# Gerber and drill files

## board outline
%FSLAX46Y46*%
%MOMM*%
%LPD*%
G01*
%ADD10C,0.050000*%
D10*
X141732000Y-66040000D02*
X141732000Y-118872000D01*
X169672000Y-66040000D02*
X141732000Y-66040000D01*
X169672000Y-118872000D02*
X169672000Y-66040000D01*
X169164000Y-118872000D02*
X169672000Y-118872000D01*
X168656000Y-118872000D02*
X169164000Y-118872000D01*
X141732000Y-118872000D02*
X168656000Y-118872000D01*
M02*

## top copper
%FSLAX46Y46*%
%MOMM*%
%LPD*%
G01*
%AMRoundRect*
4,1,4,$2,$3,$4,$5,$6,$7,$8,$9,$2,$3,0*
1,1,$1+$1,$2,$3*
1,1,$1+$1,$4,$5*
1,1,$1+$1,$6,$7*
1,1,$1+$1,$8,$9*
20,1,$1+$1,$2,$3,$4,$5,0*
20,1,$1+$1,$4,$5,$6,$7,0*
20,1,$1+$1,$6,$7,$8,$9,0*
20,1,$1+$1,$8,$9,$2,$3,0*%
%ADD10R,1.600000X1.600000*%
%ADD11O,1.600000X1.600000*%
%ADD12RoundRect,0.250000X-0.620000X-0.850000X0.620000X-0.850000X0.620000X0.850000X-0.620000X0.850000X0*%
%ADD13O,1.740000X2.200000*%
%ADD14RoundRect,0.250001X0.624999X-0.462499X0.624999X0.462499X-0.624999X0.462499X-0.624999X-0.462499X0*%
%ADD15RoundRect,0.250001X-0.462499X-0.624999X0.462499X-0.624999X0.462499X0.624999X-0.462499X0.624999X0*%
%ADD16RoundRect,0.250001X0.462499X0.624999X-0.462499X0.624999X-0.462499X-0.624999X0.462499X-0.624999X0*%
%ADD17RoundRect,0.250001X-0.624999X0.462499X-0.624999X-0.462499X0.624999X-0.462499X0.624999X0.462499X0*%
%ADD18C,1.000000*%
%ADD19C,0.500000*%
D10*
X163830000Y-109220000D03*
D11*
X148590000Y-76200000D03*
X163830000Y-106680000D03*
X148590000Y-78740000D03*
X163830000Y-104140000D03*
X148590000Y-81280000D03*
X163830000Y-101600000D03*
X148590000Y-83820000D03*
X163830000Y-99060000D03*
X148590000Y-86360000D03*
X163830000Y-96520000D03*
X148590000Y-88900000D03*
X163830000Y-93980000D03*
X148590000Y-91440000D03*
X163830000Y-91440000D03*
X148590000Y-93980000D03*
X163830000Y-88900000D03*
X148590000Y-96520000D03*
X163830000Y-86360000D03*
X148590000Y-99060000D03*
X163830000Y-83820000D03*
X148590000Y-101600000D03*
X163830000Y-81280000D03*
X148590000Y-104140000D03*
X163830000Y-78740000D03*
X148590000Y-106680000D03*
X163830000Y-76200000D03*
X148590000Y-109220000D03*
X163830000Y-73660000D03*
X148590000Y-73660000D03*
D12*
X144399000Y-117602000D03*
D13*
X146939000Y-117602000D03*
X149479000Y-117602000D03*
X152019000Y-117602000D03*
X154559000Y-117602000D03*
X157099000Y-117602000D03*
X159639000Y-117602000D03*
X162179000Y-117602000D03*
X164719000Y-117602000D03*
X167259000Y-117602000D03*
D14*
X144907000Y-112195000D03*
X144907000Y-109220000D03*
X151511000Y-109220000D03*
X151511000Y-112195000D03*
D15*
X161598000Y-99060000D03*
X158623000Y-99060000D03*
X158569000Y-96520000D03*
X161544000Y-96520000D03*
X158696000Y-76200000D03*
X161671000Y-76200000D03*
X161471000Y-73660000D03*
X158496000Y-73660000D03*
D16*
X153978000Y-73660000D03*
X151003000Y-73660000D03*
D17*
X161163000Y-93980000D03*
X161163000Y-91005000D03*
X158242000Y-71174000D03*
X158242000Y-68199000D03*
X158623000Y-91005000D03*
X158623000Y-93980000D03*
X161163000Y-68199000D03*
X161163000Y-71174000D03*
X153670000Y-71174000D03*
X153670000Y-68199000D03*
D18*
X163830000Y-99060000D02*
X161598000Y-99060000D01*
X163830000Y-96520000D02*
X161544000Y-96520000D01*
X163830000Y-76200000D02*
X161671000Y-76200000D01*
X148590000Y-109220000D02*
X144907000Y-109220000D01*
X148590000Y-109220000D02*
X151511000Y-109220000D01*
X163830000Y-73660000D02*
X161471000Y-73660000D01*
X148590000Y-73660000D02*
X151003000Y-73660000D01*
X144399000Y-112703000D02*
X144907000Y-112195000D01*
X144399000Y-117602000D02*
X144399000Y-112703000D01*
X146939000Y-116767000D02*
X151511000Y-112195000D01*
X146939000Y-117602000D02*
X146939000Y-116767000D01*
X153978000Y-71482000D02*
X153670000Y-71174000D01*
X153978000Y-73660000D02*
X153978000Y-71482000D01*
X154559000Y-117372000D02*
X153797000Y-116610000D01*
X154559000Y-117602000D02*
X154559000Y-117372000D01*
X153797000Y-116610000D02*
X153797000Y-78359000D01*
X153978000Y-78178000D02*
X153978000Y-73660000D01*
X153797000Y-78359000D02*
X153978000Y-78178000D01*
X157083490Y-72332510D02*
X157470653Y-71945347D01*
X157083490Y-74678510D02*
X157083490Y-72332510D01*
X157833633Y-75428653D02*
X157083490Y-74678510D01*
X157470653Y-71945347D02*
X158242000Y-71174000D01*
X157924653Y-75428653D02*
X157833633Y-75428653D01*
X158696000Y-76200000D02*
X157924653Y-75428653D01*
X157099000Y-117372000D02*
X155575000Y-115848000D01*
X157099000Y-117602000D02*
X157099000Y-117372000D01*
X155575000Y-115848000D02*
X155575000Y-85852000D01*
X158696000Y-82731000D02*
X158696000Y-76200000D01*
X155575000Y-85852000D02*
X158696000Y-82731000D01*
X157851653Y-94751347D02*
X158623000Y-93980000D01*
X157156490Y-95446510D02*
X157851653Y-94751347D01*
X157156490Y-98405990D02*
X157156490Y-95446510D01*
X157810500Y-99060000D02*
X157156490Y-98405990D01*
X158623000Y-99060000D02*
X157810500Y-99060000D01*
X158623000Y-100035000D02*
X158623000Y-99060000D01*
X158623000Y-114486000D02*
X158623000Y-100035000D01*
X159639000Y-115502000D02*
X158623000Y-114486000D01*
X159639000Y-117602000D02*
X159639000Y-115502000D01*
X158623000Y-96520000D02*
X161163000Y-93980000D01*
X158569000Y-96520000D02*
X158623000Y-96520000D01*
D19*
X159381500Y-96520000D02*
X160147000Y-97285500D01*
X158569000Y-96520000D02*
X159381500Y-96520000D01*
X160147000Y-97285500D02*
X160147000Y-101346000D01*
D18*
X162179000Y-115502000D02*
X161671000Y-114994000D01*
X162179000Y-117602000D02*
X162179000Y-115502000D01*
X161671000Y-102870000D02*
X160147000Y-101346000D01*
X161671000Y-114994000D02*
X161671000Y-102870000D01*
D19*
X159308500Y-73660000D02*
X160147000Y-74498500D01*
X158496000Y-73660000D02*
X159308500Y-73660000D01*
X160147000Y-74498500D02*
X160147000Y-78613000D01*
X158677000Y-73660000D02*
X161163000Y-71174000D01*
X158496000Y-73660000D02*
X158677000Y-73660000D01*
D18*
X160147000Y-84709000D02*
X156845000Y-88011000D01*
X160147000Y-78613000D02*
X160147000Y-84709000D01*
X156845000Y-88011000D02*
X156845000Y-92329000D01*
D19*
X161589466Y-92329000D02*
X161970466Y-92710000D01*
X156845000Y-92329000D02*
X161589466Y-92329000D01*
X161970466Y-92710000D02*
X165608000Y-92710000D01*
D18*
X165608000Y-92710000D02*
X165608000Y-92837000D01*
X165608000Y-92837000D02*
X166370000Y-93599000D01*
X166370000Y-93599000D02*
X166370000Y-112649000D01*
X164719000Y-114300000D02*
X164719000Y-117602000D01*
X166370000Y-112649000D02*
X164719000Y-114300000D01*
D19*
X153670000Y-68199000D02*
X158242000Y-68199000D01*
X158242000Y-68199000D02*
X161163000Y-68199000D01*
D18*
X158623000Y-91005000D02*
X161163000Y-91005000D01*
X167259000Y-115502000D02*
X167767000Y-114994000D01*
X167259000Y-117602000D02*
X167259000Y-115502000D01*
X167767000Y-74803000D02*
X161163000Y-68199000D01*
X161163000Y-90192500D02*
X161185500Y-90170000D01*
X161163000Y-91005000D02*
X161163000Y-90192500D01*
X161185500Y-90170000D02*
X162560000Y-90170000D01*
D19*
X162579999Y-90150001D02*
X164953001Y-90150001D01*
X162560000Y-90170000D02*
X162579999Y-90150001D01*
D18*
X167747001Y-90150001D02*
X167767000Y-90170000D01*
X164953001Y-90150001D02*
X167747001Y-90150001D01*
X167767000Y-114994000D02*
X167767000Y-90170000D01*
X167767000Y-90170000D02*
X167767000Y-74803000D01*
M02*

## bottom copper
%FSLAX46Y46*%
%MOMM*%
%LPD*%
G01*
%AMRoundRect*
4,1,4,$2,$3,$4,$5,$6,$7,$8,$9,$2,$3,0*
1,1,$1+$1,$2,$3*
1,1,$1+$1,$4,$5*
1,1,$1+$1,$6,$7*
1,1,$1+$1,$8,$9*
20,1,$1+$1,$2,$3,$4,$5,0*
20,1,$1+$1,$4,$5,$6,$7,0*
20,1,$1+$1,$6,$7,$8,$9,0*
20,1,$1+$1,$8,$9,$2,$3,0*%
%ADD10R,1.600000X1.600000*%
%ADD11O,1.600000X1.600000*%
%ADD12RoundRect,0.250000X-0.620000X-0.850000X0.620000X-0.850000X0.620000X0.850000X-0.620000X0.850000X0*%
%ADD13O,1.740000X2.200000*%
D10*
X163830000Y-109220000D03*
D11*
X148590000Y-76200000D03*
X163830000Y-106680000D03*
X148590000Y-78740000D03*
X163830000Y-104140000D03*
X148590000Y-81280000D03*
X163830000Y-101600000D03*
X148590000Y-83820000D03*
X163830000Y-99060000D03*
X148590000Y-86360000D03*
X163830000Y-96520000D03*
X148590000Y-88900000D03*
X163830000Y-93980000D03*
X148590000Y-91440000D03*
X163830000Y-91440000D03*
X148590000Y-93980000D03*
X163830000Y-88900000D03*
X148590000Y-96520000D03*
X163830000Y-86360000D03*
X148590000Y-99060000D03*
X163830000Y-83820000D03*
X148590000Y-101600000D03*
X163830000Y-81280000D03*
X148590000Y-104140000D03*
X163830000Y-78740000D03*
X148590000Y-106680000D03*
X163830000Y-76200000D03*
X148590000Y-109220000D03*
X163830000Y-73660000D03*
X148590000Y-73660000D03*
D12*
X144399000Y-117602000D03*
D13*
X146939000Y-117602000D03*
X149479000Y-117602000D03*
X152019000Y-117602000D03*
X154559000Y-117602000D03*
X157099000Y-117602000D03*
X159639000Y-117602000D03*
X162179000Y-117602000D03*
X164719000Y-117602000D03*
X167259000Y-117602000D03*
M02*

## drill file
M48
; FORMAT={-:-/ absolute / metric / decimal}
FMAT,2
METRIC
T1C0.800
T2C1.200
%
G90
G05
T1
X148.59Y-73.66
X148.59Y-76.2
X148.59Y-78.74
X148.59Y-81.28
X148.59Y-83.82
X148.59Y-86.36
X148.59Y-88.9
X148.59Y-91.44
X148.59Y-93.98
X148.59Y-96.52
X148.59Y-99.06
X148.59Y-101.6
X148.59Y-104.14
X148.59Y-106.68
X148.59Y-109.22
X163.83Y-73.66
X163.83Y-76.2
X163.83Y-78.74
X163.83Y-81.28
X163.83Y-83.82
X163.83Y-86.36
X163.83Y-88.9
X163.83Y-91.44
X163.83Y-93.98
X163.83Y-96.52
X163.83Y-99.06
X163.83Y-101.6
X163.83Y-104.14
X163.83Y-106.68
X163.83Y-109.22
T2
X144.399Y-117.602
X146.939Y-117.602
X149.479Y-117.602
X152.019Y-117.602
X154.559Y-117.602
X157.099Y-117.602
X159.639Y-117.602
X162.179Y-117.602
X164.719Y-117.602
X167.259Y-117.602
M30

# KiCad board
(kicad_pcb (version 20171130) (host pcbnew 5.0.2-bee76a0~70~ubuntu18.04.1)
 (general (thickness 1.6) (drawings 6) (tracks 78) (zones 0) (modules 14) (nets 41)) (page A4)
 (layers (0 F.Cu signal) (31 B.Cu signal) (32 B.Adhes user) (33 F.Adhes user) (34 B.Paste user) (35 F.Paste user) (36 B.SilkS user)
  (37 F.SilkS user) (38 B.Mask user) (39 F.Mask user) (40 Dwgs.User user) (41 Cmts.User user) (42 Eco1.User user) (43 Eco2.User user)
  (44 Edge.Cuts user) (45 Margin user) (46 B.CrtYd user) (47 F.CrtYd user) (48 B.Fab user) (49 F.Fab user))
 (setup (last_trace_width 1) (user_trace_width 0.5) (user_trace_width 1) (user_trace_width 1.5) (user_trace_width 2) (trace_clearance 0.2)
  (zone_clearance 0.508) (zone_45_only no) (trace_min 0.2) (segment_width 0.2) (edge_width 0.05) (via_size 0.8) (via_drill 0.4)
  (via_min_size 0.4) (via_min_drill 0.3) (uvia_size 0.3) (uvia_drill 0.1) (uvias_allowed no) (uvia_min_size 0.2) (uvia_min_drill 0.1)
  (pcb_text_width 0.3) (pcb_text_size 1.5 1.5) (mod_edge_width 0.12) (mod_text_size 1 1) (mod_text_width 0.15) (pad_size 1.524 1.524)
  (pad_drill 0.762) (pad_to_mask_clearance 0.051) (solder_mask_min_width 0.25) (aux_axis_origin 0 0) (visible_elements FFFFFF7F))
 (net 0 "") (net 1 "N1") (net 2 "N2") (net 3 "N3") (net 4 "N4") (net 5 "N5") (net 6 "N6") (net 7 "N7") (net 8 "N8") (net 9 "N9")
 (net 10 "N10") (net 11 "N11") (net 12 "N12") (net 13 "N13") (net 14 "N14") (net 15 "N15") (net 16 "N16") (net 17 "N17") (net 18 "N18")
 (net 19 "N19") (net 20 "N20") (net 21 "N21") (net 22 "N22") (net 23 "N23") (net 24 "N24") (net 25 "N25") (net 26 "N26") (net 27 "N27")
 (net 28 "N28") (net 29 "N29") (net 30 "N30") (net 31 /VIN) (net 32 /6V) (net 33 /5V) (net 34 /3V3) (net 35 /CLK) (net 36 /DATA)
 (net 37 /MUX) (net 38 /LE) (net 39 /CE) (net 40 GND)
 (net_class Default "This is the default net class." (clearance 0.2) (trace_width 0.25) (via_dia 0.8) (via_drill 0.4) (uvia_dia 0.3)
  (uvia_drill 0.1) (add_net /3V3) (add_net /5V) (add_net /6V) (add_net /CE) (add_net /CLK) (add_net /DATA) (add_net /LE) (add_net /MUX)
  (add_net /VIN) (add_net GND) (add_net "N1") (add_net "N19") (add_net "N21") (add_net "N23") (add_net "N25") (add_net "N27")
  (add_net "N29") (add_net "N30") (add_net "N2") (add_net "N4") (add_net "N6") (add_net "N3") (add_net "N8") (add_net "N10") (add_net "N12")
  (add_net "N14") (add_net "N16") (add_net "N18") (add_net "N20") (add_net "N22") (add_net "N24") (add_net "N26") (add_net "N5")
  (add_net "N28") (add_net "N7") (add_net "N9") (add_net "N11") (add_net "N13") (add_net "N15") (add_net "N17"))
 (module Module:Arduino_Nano (layer F.Cu) (at 163.83 109.22 180)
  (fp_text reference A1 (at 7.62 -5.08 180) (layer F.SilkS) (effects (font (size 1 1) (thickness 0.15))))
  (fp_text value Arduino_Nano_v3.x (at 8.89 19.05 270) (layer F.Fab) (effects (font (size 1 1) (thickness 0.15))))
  (pad 1 thru_hole rect (at 0 0 180) (size 1.6 1.6) (drill 0.8) (layers *.Cu *.Mask) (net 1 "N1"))
  (pad 17 thru_hole oval (at 15.24 33.02 180) (size 1.6 1.6) (drill 0.8) (layers *.Cu *.Mask) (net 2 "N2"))
  (pad 2 thru_hole oval (at 0 2.54 180) (size 1.6 1.6) (drill 0.8) (layers *.Cu *.Mask) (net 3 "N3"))
  (pad 18 thru_hole oval (at 15.24 30.48 180) (size 1.6 1.6) (drill 0.8) (layers *.Cu *.Mask) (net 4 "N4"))
  (pad 3 thru_hole oval (at 0 5.08 180) (size 1.6 1.6) (drill 0.8) (layers *.Cu *.Mask) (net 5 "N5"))
  (pad 19 thru_hole oval (at 15.24 27.94 180) (size 1.6 1.6) (drill 0.8) (layers *.Cu *.Mask) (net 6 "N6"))
  (pad 4 thru_hole oval (at 0 7.62 180) (size 1.6 1.6) (drill 0.8) (layers *.Cu *.Mask) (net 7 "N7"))
  (pad 20 thru_hole oval (at 15.24 25.4 180) (size 1.6 1.6) (drill 0.8) (layers *.Cu *.Mask) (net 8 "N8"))
  (pad 5 thru_hole oval (at 0 10.16 180) (size 1.6 1.6) (drill 0.8) (layers *.Cu *.Mask) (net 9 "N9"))
  (pad 21 thru_hole oval (at 15.24 22.86 180) (size 1.6 1.6) (drill 0.8) (layers *.Cu *.Mask) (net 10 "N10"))
  (pad 6 thru_hole oval (at 0 12.7 180) (size 1.6 1.6) (drill 0.8) (layers *.Cu *.Mask) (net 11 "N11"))
  (pad 22 thru_hole oval (at 15.24 20.32 180) (size 1.6 1.6) (drill 0.8) (layers *.Cu *.Mask) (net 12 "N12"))
  (pad 7 thru_hole oval (at 0 15.24 180) (size 1.6 1.6) (drill 0.8) (layers *.Cu *.Mask) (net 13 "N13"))
  (pad 23 thru_hole oval (at 15.24 17.78 180) (size 1.6 1.6) (drill 0.8) (layers *.Cu *.Mask) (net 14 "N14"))
  (pad 8 thru_hole oval (at 0 17.78 180) (size 1.6 1.6) (drill 0.8) (layers *.Cu *.Mask) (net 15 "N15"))
  (pad 24 thru_hole oval (at 15.24 15.24 180) (size 1.6 1.6) (drill 0.8) (layers *.Cu *.Mask) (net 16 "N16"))
  (pad 9 thru_hole oval (at 0 20.32 180) (size 1.6 1.6) (drill 0.8) (layers *.Cu *.Mask) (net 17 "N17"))
  (pad 25 thru_hole oval (at 15.24 12.7 180) (size 1.6 1.6) (drill 0.8) (layers *.Cu *.Mask) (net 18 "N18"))
  (pad 10 thru_hole oval (at 0 22.86 180) (size 1.6 1.6) (drill 0.8) (layers *.Cu *.Mask) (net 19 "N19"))
  (pad 26 thru_hole oval (at 15.24 10.16 180) (size 1.6 1.6) (drill 0.8) (layers *.Cu *.Mask) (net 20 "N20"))
  (pad 11 thru_hole oval (at 0 25.4 180) (size 1.6 1.6) (drill 0.8) (layers *.Cu *.Mask) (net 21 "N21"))
  (pad 27 thru_hole oval (at 15.24 7.62 180) (size 1.6 1.6) (drill 0.8) (layers *.Cu *.Mask) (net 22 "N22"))
  (pad 12 thru_hole oval (at 0 27.94 180) (size 1.6 1.6) (drill 0.8) (layers *.Cu *.Mask) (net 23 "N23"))
  (pad 28 thru_hole oval (at 15.24 5.08 180) (size 1.6 1.6) (drill 0.8) (layers *.Cu *.Mask) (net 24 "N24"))
  (pad 13 thru_hole oval (at 0 30.48 180) (size 1.6 1.6) (drill 0.8) (layers *.Cu *.Mask) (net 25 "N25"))
  (pad 29 thru_hole oval (at 15.24 2.54 180) (size 1.6 1.6) (drill 0.8) (layers *.Cu *.Mask) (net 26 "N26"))
  (pad 14 thru_hole oval (at 0 33.02 180) (size 1.6 1.6) (drill 0.8) (layers *.Cu *.Mask) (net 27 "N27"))
  (pad 30 thru_hole oval (at 15.24 0 180) (size 1.6 1.6) (drill 0.8) (layers *.Cu *.Mask) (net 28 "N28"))
  (pad 15 thru_hole oval (at 0 35.56 180) (size 1.6 1.6) (drill 0.8) (layers *.Cu *.Mask) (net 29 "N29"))
  (pad 16 thru_hole oval (at 15.24 35.56 180) (size 1.6 1.6) (drill 0.8) (layers *.Cu *.Mask) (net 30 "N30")))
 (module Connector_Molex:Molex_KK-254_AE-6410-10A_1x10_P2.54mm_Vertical (layer F.Cu) (at 144.399 117.602)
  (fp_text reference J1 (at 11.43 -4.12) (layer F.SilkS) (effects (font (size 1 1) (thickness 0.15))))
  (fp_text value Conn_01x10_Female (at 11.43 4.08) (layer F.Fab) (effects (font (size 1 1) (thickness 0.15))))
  (pad 1 thru_hole roundrect (at 0 0) (size 1.74 2.2) (drill 1.2) (layers *.Cu *.Mask) (roundrect_rratio 0.143678) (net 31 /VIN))
  (pad 2 thru_hole oval (at 2.54 0) (size 1.74 2.2) (drill 1.2) (layers *.Cu *.Mask) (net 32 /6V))
  (pad 3 thru_hole oval (at 5.08 0) (size 1.74 2.2) (drill 1.2) (layers *.Cu *.Mask) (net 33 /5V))
  (pad 4 thru_hole oval (at 7.62 0) (size 1.74 2.2) (drill 1.2) (layers *.Cu *.Mask) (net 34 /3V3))
  (pad 5 thru_hole oval (at 10.16 0) (size 1.74 2.2) (drill 1.2) (layers *.Cu *.Mask) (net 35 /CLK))
  (pad 6 thru_hole oval (at 12.7 0) (size 1.74 2.2) (drill 1.2) (layers *.Cu *.Mask) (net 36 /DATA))
  (pad 7 thru_hole oval (at 15.24 0) (size 1.74 2.2) (drill 1.2) (layers *.Cu *.Mask) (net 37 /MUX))
  (pad 8 thru_hole oval (at 17.78 0) (size 1.74 2.2) (drill 1.2) (layers *.Cu *.Mask) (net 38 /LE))
  (pad 9 thru_hole oval (at 20.32 0) (size 1.74 2.2) (drill 1.2) (layers *.Cu *.Mask) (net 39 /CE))
  (pad 10 thru_hole oval (at 22.86 0) (size 1.74 2.2) (drill 1.2) (layers *.Cu *.Mask) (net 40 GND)))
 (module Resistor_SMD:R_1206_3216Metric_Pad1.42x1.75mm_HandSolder (layer F.Cu) (at 144.907 110.7075 90)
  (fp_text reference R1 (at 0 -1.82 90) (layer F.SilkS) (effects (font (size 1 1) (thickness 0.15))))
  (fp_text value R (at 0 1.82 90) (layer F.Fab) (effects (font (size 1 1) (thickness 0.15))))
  (pad 1 smd roundrect (at -1.4875 0 90) (size 1.425 1.75) (layers F.Cu F.Paste F.Mask) (roundrect_rratio 0.175439) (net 31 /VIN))
  (pad 2 smd roundrect (at 1.4875 0 90) (size 1.425 1.75) (layers F.Cu F.Paste F.Mask) (roundrect_rratio 0.175439) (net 28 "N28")))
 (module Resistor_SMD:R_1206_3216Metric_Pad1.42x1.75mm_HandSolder (layer F.Cu) (at 151.511 110.7075 90)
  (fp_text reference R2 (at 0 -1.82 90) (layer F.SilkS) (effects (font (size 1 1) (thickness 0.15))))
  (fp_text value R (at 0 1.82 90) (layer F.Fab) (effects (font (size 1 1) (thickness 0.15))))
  (pad 2 smd roundrect (at 1.4875 0 90) (size 1.425 1.75) (layers F.Cu F.Paste F.Mask) (roundrect_rratio 0.175439) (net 28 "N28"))
  (pad 1 smd roundrect (at -1.4875 0 90) (size 1.425 1.75) (layers F.Cu F.Paste F.Mask) (roundrect_rratio 0.175439) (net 32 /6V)))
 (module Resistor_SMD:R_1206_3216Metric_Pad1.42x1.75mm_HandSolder (layer F.Cu) (at 160.1105 99.06)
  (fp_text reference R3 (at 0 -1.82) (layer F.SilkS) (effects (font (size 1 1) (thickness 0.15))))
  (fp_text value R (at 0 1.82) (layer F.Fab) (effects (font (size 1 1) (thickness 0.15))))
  (pad 2 smd roundrect (at 1.4875 0) (size 1.425 1.75) (layers F.Cu F.Paste F.Mask) (roundrect_rratio 0.175439) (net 9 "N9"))
  (pad 1 smd roundrect (at -1.4875 0) (size 1.425 1.75) (layers F.Cu F.Paste F.Mask) (roundrect_rratio 0.175439) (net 37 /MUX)))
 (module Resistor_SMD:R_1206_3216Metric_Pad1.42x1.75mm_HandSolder (layer F.Cu) (at 160.0565 96.52)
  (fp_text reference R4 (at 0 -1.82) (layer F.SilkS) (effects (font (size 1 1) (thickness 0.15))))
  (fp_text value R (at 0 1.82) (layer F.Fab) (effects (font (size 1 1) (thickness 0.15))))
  (pad 1 smd roundrect (at -1.4875 0) (size 1.425 1.75) (layers F.Cu F.Paste F.Mask) (roundrect_rratio 0.175439) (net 38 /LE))
  (pad 2 smd roundrect (at 1.4875 0) (size 1.425 1.75) (layers F.Cu F.Paste F.Mask) (roundrect_rratio 0.175439) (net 11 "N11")))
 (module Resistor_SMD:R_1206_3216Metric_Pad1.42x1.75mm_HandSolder (layer F.Cu) (at 160.1835 76.2)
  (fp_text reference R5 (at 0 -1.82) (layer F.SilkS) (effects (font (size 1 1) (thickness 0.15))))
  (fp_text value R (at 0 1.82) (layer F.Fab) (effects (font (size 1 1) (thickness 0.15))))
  (pad 1 smd roundrect (at -1.4875 0) (size 1.425 1.75) (layers F.Cu F.Paste F.Mask) (roundrect_rratio 0.175439) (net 36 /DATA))
  (pad 2 smd roundrect (at 1.4875 0) (size 1.425 1.75) (layers F.Cu F.Paste F.Mask) (roundrect_rratio 0.175439) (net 27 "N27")))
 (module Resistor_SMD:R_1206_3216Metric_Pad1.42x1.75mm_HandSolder (layer F.Cu) (at 159.9835 73.66)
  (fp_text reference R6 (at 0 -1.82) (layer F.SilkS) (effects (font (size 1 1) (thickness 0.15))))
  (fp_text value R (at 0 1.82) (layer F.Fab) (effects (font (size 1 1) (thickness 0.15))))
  (pad 2 smd roundrect (at 1.4875 0) (size 1.425 1.75) (layers F.Cu F.Paste F.Mask) (roundrect_rratio 0.175439) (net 29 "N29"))
  (pad 1 smd roundrect (at -1.4875 0) (size 1.425 1.75) (layers F.Cu F.Paste F.Mask) (roundrect_rratio 0.175439) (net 39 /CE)))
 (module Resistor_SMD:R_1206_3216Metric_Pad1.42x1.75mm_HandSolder (layer F.Cu) (at 152.4905 73.66 180)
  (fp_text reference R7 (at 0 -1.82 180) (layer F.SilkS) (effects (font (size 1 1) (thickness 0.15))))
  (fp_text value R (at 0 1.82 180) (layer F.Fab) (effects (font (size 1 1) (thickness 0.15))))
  (pad 1 smd roundrect (at -1.4875 0 180) (size 1.425 1.75) (layers F.Cu F.Paste F.Mask) (roundrect_rratio 0.175439) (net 35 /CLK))
  (pad 2 smd roundrect (at 1.4875 0 180) (size 1.425 1.75) (layers F.Cu F.Paste F.Mask) (roundrect_rratio 0.175439) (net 30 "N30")))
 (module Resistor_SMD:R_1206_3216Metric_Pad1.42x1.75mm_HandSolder (layer F.Cu) (at 161.163 92.4925 270)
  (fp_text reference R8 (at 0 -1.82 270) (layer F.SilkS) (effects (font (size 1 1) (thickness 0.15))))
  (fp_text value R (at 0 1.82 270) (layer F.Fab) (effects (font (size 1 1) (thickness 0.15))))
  (pad 2 smd roundrect (at 1.4875 0 270) (size 1.425 1.75) (layers F.Cu F.Paste F.Mask) (roundrect_rratio 0.175439) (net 38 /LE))
  (pad 1 smd roundrect (at -1.4875 0 270) (size 1.425 1.75) (layers F.Cu F.Paste F.Mask) (roundrect_rratio 0.175439) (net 40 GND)))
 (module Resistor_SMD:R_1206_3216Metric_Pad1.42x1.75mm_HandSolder (layer F.Cu) (at 158.242 69.6865 270)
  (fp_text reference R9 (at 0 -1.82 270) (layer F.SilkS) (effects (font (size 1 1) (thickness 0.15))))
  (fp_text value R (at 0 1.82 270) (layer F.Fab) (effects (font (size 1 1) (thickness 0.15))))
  (pad 2 smd roundrect (at 1.4875 0 270) (size 1.425 1.75) (layers F.Cu F.Paste F.Mask) (roundrect_rratio 0.175439) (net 36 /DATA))
  (pad 1 smd roundrect (at -1.4875 0 270) (size 1.425 1.75) (layers F.Cu F.Paste F.Mask) (roundrect_rratio 0.175439) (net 40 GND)))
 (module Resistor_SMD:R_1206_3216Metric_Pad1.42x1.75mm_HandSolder (layer F.Cu) (at 158.623 92.4925 270)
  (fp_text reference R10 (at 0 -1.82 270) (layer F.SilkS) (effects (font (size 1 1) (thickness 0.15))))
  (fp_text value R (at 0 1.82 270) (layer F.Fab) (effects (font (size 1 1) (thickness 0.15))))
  (pad 1 smd roundrect (at -1.4875 0 270) (size 1.425 1.75) (layers F.Cu F.Paste F.Mask) (roundrect_rratio 0.175439) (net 40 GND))
  (pad 2 smd roundrect (at 1.4875 0 270) (size 1.425 1.75) (layers F.Cu F.Paste F.Mask) (roundrect_rratio 0.175439) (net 37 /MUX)))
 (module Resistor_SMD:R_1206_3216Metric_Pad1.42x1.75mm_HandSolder (layer F.Cu) (at 161.163 69.6865 270)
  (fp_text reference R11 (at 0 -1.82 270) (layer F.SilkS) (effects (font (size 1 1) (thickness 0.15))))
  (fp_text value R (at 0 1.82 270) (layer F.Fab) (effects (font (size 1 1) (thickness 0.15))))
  (pad 1 smd roundrect (at -1.4875 0 270) (size 1.425 1.75) (layers F.Cu F.Paste F.Mask) (roundrect_rratio 0.175439) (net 40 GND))
  (pad 2 smd roundrect (at 1.4875 0 270) (size 1.425 1.75) (layers F.Cu F.Paste F.Mask) (roundrect_rratio 0.175439) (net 39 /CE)))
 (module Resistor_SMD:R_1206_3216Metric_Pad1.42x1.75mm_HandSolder (layer F.Cu) (at 153.67 69.6865 270)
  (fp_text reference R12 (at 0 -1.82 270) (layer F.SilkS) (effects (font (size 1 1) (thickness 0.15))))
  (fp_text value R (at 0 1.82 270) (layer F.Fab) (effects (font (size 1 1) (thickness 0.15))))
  (pad 2 smd roundrect (at 1.4875 0 270) (size 1.425 1.75) (layers F.Cu F.Paste F.Mask) (roundrect_rratio 0.175439) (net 35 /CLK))
  (pad 1 smd roundrect (at -1.4875 0 270) (size 1.425 1.75) (layers F.Cu F.Paste F.Mask) (roundrect_rratio 0.175439) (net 40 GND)))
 (gr_line (start 141.732 66.04) (end 141.732 118.872) (layer Edge.Cuts) (width 0.05))
 (gr_line (start 169.672 66.04) (end 141.732 66.04) (layer Edge.Cuts) (width 0.05))
 (gr_line (start 169.672 118.872) (end 169.672 66.04) (layer Edge.Cuts) (width 0.05))
 (gr_line (start 169.164 118.872) (end 169.672 118.872) (layer Edge.Cuts) (width 0.05))
 (gr_line (start 168.656 118.872) (end 169.164 118.872) (layer Edge.Cuts) (width 0.05))
 (gr_line (start 141.732 118.872) (end 168.656 118.872) (layer Edge.Cuts) (width 0.05))
 (segment (start 163.83 99.06) (end 161.598 99.06) (width 1) (layer F.Cu) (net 9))
 (segment (start 163.83 96.52) (end 161.544 96.52) (width 1) (layer F.Cu) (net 11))
 (segment (start 163.83 76.2) (end 161.671 76.2) (width 1) (layer F.Cu) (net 27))
 (segment (start 148.59 109.22) (end 144.907 109.22) (width 1) (layer F.Cu) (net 28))
 (segment (start 148.59 109.22) (end 151.511 109.22) (width 1) (layer F.Cu) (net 28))
 (segment (start 163.83 73.66) (end 161.471 73.66) (width 1) (layer F.Cu) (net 29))
 (segment (start 148.59 73.66) (end 151.003 73.66) (width 1) (layer F.Cu) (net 30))
 (segment (start 144.399 112.703) (end 144.907 112.195) (width 1) (layer F.Cu) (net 31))
 (segment (start 144.399 117.602) (end 144.399 112.703) (width 1) (layer F.Cu) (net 31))
 (segment (start 146.939 116.767) (end 151.511 112.195) (width 1) (layer F.Cu) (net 32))
 (segment (start 146.939 117.602) (end 146.939 116.767) (width 1) (layer F.Cu) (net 32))
 (segment (start 153.978 71.482) (end 153.67 71.174) (width 1) (layer F.Cu) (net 35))
 (segment (start 153.978 73.66) (end 153.978 71.482) (width 1) (layer F.Cu) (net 35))
 (segment (start 154.559 117.372) (end 153.797 116.61) (width 1) (layer F.Cu) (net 35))
 (segment (start 154.559 117.602) (end 154.559 117.372) (width 1) (layer F.Cu) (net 35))
 (segment (start 153.797 116.61) (end 153.797 78.359) (width 1) (layer F.Cu) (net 35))
 (segment (start 153.978 78.178) (end 153.978 73.66) (width 1) (layer F.Cu) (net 35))
 (segment (start 153.797 78.359) (end 153.978 78.178) (width 1) (layer F.Cu) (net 35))
 (segment (start 157.08349 72.33251) (end 157.470653 71.945347) (width 1) (layer F.Cu) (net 36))
 (segment (start 157.08349 74.67851) (end 157.08349 72.33251) (width 1) (layer F.Cu) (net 36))
 (segment (start 157.833633 75.428653) (end 157.08349 74.67851) (width 1) (layer F.Cu) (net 36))
 (segment (start 157.470653 71.945347) (end 158.242 71.174) (width 1) (layer F.Cu) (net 36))
 (segment (start 157.924653 75.428653) (end 157.833633 75.428653) (width 1) (layer F.Cu) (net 36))
 (segment (start 158.696 76.2) (end 157.924653 75.428653) (width 1) (layer F.Cu) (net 36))
 (segment (start 157.099 117.372) (end 155.575 115.848) (width 1) (layer F.Cu) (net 36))
 (segment (start 157.099 117.602) (end 157.099 117.372) (width 1) (layer F.Cu) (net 36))
 (segment (start 155.575 115.848) (end 155.575 85.852) (width 1) (layer F.Cu) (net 36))
 (segment (start 158.696 82.731) (end 158.696 76.2) (width 1) (layer F.Cu) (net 36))
 (segment (start 155.575 85.852) (end 158.696 82.731) (width 1) (layer F.Cu) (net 36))
 (segment (start 157.851653 94.751347) (end 158.623 93.98) (width 1) (layer F.Cu) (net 37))
 (segment (start 157.15649 95.44651) (end 157.851653 94.751347) (width 1) (layer F.Cu) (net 37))
 (segment (start 157.15649 98.40599) (end 157.15649 95.44651) (width 1) (layer F.Cu) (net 37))
 (segment (start 157.8105 99.06) (end 157.15649 98.40599) (width 1) (layer F.Cu) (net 37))
 (segment (start 158.623 99.06) (end 157.8105 99.06) (width 1) (layer F.Cu) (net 37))
 (segment (start 158.623 100.035) (end 158.623 99.06) (width 1) (layer F.Cu) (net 37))
 (segment (start 158.623 114.486) (end 158.623 100.035) (width 1) (layer F.Cu) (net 37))
 (segment (start 159.639 115.502) (end 158.623 114.486) (width 1) (layer F.Cu) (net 37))
 (segment (start 159.639 117.602) (end 159.639 115.502) (width 1) (layer F.Cu) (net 37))
 (segment (start 158.623 96.52) (end 161.163 93.98) (width 1) (layer F.Cu) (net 38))
 (segment (start 158.569 96.52) (end 158.623 96.52) (width 1) (layer F.Cu) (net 38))
 (segment (start 159.3815 96.52) (end 160.147 97.2855) (width 0.5) (layer F.Cu) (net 38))
 (segment (start 158.569 96.52) (end 159.3815 96.52) (width 0.5) (layer F.Cu) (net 38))
 (segment (start 160.147 97.2855) (end 160.147 101.346) (width 0.5) (layer F.Cu) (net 38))
 (segment (start 162.179 115.502) (end 161.671 114.994) (width 1) (layer F.Cu) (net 38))
 (segment (start 162.179 117.602) (end 162.179 115.502) (width 1) (layer F.Cu) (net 38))
 (segment (start 161.671 102.87) (end 160.147 101.346) (width 1) (layer F.Cu) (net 38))
 (segment (start 161.671 114.994) (end 161.671 102.87) (width 1) (layer F.Cu) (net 38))
 (segment (start 159.3085 73.66) (end 160.147 74.4985) (width 0.5) (layer F.Cu) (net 39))
 (segment (start 158.496 73.66) (end 159.3085 73.66) (width 0.5) (layer F.Cu) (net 39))
 (segment (start 160.147 74.4985) (end 160.147 78.613) (width 0.5) (layer F.Cu) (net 39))
 (segment (start 158.677 73.66) (end 161.163 71.174) (width 0.5) (layer F.Cu) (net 39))
 (segment (start 158.496 73.66) (end 158.677 73.66) (width 0.5) (layer F.Cu) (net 39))
 (segment (start 160.147 84.709) (end 156.845 88.011) (width 1) (layer F.Cu) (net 39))
 (segment (start 160.147 78.613) (end 160.147 84.709) (width 1) (layer F.Cu) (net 39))
 (segment (start 156.845 88.011) (end 156.845 92.329) (width 1) (layer F.Cu) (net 39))
 (segment (start 161.589466 92.329) (end 161.970466 92.71) (width 0.5) (layer F.Cu) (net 39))
 (segment (start 156.845 92.329) (end 161.589466 92.329) (width 0.5) (layer F.Cu) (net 39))
 (segment (start 161.970466 92.71) (end 165.608 92.71) (width 0.5) (layer F.Cu) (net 39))
 (segment (start 165.608 92.71) (end 165.608 92.837) (width 1) (layer F.Cu) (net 39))
 (segment (start 165.608 92.837) (end 166.37 93.599) (width 1) (layer F.Cu) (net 39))
 (segment (start 166.37 93.599) (end 166.37 112.649) (width 1) (layer F.Cu) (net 39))
 (segment (start 164.719 114.3) (end 164.719 117.602) (width 1) (layer F.Cu) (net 39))
 (segment (start 166.37 112.649) (end 164.719 114.3) (width 1) (layer F.Cu) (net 39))
 (segment (start 153.67 68.199) (end 158.242 68.199) (width 0.5) (layer F.Cu) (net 40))
 (segment (start 158.242 68.199) (end 161.163 68.199) (width 0.5) (layer F.Cu) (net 40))
 (segment (start 158.623 91.005) (end 161.163 91.005) (width 1) (layer F.Cu) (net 40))
 (segment (start 167.259 115.502) (end 167.767 114.994) (width 1) (layer F.Cu) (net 40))
 (segment (start 167.259 117.602) (end 167.259 115.502) (width 1) (layer F.Cu) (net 40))
 (segment (start 167.767 74.803) (end 161.163 68.199) (width 1) (layer F.Cu) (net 40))
 (segment (start 161.163 90.1925) (end 161.1855 90.17) (width 1) (layer F.Cu) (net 40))
 (segment (start 161.163 91.005) (end 161.163 90.1925) (width 1) (layer F.Cu) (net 40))
 (segment (start 161.1855 90.17) (end 162.56 90.17) (width 1) (layer F.Cu) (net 40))
 (segment (start 162.579999 90.150001) (end 164.953001 90.150001) (width 0.5) (layer F.Cu) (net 40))
 (segment (start 162.56 90.17) (end 162.579999 90.150001) (width 0.5) (layer F.Cu) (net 40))
 (segment (start 167.747001 90.150001) (end 167.767 90.17) (width 1) (layer F.Cu) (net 40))
 (segment (start 164.953001 90.150001) (end 167.747001 90.150001) (width 1) (layer F.Cu) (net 40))
 (segment (start 167.767 114.994) (end 167.767 90.17) (width 1) (layer F.Cu) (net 40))
 (segment (start 167.767 90.17) (end 167.767 74.803) (width 1) (layer F.Cu) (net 40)))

